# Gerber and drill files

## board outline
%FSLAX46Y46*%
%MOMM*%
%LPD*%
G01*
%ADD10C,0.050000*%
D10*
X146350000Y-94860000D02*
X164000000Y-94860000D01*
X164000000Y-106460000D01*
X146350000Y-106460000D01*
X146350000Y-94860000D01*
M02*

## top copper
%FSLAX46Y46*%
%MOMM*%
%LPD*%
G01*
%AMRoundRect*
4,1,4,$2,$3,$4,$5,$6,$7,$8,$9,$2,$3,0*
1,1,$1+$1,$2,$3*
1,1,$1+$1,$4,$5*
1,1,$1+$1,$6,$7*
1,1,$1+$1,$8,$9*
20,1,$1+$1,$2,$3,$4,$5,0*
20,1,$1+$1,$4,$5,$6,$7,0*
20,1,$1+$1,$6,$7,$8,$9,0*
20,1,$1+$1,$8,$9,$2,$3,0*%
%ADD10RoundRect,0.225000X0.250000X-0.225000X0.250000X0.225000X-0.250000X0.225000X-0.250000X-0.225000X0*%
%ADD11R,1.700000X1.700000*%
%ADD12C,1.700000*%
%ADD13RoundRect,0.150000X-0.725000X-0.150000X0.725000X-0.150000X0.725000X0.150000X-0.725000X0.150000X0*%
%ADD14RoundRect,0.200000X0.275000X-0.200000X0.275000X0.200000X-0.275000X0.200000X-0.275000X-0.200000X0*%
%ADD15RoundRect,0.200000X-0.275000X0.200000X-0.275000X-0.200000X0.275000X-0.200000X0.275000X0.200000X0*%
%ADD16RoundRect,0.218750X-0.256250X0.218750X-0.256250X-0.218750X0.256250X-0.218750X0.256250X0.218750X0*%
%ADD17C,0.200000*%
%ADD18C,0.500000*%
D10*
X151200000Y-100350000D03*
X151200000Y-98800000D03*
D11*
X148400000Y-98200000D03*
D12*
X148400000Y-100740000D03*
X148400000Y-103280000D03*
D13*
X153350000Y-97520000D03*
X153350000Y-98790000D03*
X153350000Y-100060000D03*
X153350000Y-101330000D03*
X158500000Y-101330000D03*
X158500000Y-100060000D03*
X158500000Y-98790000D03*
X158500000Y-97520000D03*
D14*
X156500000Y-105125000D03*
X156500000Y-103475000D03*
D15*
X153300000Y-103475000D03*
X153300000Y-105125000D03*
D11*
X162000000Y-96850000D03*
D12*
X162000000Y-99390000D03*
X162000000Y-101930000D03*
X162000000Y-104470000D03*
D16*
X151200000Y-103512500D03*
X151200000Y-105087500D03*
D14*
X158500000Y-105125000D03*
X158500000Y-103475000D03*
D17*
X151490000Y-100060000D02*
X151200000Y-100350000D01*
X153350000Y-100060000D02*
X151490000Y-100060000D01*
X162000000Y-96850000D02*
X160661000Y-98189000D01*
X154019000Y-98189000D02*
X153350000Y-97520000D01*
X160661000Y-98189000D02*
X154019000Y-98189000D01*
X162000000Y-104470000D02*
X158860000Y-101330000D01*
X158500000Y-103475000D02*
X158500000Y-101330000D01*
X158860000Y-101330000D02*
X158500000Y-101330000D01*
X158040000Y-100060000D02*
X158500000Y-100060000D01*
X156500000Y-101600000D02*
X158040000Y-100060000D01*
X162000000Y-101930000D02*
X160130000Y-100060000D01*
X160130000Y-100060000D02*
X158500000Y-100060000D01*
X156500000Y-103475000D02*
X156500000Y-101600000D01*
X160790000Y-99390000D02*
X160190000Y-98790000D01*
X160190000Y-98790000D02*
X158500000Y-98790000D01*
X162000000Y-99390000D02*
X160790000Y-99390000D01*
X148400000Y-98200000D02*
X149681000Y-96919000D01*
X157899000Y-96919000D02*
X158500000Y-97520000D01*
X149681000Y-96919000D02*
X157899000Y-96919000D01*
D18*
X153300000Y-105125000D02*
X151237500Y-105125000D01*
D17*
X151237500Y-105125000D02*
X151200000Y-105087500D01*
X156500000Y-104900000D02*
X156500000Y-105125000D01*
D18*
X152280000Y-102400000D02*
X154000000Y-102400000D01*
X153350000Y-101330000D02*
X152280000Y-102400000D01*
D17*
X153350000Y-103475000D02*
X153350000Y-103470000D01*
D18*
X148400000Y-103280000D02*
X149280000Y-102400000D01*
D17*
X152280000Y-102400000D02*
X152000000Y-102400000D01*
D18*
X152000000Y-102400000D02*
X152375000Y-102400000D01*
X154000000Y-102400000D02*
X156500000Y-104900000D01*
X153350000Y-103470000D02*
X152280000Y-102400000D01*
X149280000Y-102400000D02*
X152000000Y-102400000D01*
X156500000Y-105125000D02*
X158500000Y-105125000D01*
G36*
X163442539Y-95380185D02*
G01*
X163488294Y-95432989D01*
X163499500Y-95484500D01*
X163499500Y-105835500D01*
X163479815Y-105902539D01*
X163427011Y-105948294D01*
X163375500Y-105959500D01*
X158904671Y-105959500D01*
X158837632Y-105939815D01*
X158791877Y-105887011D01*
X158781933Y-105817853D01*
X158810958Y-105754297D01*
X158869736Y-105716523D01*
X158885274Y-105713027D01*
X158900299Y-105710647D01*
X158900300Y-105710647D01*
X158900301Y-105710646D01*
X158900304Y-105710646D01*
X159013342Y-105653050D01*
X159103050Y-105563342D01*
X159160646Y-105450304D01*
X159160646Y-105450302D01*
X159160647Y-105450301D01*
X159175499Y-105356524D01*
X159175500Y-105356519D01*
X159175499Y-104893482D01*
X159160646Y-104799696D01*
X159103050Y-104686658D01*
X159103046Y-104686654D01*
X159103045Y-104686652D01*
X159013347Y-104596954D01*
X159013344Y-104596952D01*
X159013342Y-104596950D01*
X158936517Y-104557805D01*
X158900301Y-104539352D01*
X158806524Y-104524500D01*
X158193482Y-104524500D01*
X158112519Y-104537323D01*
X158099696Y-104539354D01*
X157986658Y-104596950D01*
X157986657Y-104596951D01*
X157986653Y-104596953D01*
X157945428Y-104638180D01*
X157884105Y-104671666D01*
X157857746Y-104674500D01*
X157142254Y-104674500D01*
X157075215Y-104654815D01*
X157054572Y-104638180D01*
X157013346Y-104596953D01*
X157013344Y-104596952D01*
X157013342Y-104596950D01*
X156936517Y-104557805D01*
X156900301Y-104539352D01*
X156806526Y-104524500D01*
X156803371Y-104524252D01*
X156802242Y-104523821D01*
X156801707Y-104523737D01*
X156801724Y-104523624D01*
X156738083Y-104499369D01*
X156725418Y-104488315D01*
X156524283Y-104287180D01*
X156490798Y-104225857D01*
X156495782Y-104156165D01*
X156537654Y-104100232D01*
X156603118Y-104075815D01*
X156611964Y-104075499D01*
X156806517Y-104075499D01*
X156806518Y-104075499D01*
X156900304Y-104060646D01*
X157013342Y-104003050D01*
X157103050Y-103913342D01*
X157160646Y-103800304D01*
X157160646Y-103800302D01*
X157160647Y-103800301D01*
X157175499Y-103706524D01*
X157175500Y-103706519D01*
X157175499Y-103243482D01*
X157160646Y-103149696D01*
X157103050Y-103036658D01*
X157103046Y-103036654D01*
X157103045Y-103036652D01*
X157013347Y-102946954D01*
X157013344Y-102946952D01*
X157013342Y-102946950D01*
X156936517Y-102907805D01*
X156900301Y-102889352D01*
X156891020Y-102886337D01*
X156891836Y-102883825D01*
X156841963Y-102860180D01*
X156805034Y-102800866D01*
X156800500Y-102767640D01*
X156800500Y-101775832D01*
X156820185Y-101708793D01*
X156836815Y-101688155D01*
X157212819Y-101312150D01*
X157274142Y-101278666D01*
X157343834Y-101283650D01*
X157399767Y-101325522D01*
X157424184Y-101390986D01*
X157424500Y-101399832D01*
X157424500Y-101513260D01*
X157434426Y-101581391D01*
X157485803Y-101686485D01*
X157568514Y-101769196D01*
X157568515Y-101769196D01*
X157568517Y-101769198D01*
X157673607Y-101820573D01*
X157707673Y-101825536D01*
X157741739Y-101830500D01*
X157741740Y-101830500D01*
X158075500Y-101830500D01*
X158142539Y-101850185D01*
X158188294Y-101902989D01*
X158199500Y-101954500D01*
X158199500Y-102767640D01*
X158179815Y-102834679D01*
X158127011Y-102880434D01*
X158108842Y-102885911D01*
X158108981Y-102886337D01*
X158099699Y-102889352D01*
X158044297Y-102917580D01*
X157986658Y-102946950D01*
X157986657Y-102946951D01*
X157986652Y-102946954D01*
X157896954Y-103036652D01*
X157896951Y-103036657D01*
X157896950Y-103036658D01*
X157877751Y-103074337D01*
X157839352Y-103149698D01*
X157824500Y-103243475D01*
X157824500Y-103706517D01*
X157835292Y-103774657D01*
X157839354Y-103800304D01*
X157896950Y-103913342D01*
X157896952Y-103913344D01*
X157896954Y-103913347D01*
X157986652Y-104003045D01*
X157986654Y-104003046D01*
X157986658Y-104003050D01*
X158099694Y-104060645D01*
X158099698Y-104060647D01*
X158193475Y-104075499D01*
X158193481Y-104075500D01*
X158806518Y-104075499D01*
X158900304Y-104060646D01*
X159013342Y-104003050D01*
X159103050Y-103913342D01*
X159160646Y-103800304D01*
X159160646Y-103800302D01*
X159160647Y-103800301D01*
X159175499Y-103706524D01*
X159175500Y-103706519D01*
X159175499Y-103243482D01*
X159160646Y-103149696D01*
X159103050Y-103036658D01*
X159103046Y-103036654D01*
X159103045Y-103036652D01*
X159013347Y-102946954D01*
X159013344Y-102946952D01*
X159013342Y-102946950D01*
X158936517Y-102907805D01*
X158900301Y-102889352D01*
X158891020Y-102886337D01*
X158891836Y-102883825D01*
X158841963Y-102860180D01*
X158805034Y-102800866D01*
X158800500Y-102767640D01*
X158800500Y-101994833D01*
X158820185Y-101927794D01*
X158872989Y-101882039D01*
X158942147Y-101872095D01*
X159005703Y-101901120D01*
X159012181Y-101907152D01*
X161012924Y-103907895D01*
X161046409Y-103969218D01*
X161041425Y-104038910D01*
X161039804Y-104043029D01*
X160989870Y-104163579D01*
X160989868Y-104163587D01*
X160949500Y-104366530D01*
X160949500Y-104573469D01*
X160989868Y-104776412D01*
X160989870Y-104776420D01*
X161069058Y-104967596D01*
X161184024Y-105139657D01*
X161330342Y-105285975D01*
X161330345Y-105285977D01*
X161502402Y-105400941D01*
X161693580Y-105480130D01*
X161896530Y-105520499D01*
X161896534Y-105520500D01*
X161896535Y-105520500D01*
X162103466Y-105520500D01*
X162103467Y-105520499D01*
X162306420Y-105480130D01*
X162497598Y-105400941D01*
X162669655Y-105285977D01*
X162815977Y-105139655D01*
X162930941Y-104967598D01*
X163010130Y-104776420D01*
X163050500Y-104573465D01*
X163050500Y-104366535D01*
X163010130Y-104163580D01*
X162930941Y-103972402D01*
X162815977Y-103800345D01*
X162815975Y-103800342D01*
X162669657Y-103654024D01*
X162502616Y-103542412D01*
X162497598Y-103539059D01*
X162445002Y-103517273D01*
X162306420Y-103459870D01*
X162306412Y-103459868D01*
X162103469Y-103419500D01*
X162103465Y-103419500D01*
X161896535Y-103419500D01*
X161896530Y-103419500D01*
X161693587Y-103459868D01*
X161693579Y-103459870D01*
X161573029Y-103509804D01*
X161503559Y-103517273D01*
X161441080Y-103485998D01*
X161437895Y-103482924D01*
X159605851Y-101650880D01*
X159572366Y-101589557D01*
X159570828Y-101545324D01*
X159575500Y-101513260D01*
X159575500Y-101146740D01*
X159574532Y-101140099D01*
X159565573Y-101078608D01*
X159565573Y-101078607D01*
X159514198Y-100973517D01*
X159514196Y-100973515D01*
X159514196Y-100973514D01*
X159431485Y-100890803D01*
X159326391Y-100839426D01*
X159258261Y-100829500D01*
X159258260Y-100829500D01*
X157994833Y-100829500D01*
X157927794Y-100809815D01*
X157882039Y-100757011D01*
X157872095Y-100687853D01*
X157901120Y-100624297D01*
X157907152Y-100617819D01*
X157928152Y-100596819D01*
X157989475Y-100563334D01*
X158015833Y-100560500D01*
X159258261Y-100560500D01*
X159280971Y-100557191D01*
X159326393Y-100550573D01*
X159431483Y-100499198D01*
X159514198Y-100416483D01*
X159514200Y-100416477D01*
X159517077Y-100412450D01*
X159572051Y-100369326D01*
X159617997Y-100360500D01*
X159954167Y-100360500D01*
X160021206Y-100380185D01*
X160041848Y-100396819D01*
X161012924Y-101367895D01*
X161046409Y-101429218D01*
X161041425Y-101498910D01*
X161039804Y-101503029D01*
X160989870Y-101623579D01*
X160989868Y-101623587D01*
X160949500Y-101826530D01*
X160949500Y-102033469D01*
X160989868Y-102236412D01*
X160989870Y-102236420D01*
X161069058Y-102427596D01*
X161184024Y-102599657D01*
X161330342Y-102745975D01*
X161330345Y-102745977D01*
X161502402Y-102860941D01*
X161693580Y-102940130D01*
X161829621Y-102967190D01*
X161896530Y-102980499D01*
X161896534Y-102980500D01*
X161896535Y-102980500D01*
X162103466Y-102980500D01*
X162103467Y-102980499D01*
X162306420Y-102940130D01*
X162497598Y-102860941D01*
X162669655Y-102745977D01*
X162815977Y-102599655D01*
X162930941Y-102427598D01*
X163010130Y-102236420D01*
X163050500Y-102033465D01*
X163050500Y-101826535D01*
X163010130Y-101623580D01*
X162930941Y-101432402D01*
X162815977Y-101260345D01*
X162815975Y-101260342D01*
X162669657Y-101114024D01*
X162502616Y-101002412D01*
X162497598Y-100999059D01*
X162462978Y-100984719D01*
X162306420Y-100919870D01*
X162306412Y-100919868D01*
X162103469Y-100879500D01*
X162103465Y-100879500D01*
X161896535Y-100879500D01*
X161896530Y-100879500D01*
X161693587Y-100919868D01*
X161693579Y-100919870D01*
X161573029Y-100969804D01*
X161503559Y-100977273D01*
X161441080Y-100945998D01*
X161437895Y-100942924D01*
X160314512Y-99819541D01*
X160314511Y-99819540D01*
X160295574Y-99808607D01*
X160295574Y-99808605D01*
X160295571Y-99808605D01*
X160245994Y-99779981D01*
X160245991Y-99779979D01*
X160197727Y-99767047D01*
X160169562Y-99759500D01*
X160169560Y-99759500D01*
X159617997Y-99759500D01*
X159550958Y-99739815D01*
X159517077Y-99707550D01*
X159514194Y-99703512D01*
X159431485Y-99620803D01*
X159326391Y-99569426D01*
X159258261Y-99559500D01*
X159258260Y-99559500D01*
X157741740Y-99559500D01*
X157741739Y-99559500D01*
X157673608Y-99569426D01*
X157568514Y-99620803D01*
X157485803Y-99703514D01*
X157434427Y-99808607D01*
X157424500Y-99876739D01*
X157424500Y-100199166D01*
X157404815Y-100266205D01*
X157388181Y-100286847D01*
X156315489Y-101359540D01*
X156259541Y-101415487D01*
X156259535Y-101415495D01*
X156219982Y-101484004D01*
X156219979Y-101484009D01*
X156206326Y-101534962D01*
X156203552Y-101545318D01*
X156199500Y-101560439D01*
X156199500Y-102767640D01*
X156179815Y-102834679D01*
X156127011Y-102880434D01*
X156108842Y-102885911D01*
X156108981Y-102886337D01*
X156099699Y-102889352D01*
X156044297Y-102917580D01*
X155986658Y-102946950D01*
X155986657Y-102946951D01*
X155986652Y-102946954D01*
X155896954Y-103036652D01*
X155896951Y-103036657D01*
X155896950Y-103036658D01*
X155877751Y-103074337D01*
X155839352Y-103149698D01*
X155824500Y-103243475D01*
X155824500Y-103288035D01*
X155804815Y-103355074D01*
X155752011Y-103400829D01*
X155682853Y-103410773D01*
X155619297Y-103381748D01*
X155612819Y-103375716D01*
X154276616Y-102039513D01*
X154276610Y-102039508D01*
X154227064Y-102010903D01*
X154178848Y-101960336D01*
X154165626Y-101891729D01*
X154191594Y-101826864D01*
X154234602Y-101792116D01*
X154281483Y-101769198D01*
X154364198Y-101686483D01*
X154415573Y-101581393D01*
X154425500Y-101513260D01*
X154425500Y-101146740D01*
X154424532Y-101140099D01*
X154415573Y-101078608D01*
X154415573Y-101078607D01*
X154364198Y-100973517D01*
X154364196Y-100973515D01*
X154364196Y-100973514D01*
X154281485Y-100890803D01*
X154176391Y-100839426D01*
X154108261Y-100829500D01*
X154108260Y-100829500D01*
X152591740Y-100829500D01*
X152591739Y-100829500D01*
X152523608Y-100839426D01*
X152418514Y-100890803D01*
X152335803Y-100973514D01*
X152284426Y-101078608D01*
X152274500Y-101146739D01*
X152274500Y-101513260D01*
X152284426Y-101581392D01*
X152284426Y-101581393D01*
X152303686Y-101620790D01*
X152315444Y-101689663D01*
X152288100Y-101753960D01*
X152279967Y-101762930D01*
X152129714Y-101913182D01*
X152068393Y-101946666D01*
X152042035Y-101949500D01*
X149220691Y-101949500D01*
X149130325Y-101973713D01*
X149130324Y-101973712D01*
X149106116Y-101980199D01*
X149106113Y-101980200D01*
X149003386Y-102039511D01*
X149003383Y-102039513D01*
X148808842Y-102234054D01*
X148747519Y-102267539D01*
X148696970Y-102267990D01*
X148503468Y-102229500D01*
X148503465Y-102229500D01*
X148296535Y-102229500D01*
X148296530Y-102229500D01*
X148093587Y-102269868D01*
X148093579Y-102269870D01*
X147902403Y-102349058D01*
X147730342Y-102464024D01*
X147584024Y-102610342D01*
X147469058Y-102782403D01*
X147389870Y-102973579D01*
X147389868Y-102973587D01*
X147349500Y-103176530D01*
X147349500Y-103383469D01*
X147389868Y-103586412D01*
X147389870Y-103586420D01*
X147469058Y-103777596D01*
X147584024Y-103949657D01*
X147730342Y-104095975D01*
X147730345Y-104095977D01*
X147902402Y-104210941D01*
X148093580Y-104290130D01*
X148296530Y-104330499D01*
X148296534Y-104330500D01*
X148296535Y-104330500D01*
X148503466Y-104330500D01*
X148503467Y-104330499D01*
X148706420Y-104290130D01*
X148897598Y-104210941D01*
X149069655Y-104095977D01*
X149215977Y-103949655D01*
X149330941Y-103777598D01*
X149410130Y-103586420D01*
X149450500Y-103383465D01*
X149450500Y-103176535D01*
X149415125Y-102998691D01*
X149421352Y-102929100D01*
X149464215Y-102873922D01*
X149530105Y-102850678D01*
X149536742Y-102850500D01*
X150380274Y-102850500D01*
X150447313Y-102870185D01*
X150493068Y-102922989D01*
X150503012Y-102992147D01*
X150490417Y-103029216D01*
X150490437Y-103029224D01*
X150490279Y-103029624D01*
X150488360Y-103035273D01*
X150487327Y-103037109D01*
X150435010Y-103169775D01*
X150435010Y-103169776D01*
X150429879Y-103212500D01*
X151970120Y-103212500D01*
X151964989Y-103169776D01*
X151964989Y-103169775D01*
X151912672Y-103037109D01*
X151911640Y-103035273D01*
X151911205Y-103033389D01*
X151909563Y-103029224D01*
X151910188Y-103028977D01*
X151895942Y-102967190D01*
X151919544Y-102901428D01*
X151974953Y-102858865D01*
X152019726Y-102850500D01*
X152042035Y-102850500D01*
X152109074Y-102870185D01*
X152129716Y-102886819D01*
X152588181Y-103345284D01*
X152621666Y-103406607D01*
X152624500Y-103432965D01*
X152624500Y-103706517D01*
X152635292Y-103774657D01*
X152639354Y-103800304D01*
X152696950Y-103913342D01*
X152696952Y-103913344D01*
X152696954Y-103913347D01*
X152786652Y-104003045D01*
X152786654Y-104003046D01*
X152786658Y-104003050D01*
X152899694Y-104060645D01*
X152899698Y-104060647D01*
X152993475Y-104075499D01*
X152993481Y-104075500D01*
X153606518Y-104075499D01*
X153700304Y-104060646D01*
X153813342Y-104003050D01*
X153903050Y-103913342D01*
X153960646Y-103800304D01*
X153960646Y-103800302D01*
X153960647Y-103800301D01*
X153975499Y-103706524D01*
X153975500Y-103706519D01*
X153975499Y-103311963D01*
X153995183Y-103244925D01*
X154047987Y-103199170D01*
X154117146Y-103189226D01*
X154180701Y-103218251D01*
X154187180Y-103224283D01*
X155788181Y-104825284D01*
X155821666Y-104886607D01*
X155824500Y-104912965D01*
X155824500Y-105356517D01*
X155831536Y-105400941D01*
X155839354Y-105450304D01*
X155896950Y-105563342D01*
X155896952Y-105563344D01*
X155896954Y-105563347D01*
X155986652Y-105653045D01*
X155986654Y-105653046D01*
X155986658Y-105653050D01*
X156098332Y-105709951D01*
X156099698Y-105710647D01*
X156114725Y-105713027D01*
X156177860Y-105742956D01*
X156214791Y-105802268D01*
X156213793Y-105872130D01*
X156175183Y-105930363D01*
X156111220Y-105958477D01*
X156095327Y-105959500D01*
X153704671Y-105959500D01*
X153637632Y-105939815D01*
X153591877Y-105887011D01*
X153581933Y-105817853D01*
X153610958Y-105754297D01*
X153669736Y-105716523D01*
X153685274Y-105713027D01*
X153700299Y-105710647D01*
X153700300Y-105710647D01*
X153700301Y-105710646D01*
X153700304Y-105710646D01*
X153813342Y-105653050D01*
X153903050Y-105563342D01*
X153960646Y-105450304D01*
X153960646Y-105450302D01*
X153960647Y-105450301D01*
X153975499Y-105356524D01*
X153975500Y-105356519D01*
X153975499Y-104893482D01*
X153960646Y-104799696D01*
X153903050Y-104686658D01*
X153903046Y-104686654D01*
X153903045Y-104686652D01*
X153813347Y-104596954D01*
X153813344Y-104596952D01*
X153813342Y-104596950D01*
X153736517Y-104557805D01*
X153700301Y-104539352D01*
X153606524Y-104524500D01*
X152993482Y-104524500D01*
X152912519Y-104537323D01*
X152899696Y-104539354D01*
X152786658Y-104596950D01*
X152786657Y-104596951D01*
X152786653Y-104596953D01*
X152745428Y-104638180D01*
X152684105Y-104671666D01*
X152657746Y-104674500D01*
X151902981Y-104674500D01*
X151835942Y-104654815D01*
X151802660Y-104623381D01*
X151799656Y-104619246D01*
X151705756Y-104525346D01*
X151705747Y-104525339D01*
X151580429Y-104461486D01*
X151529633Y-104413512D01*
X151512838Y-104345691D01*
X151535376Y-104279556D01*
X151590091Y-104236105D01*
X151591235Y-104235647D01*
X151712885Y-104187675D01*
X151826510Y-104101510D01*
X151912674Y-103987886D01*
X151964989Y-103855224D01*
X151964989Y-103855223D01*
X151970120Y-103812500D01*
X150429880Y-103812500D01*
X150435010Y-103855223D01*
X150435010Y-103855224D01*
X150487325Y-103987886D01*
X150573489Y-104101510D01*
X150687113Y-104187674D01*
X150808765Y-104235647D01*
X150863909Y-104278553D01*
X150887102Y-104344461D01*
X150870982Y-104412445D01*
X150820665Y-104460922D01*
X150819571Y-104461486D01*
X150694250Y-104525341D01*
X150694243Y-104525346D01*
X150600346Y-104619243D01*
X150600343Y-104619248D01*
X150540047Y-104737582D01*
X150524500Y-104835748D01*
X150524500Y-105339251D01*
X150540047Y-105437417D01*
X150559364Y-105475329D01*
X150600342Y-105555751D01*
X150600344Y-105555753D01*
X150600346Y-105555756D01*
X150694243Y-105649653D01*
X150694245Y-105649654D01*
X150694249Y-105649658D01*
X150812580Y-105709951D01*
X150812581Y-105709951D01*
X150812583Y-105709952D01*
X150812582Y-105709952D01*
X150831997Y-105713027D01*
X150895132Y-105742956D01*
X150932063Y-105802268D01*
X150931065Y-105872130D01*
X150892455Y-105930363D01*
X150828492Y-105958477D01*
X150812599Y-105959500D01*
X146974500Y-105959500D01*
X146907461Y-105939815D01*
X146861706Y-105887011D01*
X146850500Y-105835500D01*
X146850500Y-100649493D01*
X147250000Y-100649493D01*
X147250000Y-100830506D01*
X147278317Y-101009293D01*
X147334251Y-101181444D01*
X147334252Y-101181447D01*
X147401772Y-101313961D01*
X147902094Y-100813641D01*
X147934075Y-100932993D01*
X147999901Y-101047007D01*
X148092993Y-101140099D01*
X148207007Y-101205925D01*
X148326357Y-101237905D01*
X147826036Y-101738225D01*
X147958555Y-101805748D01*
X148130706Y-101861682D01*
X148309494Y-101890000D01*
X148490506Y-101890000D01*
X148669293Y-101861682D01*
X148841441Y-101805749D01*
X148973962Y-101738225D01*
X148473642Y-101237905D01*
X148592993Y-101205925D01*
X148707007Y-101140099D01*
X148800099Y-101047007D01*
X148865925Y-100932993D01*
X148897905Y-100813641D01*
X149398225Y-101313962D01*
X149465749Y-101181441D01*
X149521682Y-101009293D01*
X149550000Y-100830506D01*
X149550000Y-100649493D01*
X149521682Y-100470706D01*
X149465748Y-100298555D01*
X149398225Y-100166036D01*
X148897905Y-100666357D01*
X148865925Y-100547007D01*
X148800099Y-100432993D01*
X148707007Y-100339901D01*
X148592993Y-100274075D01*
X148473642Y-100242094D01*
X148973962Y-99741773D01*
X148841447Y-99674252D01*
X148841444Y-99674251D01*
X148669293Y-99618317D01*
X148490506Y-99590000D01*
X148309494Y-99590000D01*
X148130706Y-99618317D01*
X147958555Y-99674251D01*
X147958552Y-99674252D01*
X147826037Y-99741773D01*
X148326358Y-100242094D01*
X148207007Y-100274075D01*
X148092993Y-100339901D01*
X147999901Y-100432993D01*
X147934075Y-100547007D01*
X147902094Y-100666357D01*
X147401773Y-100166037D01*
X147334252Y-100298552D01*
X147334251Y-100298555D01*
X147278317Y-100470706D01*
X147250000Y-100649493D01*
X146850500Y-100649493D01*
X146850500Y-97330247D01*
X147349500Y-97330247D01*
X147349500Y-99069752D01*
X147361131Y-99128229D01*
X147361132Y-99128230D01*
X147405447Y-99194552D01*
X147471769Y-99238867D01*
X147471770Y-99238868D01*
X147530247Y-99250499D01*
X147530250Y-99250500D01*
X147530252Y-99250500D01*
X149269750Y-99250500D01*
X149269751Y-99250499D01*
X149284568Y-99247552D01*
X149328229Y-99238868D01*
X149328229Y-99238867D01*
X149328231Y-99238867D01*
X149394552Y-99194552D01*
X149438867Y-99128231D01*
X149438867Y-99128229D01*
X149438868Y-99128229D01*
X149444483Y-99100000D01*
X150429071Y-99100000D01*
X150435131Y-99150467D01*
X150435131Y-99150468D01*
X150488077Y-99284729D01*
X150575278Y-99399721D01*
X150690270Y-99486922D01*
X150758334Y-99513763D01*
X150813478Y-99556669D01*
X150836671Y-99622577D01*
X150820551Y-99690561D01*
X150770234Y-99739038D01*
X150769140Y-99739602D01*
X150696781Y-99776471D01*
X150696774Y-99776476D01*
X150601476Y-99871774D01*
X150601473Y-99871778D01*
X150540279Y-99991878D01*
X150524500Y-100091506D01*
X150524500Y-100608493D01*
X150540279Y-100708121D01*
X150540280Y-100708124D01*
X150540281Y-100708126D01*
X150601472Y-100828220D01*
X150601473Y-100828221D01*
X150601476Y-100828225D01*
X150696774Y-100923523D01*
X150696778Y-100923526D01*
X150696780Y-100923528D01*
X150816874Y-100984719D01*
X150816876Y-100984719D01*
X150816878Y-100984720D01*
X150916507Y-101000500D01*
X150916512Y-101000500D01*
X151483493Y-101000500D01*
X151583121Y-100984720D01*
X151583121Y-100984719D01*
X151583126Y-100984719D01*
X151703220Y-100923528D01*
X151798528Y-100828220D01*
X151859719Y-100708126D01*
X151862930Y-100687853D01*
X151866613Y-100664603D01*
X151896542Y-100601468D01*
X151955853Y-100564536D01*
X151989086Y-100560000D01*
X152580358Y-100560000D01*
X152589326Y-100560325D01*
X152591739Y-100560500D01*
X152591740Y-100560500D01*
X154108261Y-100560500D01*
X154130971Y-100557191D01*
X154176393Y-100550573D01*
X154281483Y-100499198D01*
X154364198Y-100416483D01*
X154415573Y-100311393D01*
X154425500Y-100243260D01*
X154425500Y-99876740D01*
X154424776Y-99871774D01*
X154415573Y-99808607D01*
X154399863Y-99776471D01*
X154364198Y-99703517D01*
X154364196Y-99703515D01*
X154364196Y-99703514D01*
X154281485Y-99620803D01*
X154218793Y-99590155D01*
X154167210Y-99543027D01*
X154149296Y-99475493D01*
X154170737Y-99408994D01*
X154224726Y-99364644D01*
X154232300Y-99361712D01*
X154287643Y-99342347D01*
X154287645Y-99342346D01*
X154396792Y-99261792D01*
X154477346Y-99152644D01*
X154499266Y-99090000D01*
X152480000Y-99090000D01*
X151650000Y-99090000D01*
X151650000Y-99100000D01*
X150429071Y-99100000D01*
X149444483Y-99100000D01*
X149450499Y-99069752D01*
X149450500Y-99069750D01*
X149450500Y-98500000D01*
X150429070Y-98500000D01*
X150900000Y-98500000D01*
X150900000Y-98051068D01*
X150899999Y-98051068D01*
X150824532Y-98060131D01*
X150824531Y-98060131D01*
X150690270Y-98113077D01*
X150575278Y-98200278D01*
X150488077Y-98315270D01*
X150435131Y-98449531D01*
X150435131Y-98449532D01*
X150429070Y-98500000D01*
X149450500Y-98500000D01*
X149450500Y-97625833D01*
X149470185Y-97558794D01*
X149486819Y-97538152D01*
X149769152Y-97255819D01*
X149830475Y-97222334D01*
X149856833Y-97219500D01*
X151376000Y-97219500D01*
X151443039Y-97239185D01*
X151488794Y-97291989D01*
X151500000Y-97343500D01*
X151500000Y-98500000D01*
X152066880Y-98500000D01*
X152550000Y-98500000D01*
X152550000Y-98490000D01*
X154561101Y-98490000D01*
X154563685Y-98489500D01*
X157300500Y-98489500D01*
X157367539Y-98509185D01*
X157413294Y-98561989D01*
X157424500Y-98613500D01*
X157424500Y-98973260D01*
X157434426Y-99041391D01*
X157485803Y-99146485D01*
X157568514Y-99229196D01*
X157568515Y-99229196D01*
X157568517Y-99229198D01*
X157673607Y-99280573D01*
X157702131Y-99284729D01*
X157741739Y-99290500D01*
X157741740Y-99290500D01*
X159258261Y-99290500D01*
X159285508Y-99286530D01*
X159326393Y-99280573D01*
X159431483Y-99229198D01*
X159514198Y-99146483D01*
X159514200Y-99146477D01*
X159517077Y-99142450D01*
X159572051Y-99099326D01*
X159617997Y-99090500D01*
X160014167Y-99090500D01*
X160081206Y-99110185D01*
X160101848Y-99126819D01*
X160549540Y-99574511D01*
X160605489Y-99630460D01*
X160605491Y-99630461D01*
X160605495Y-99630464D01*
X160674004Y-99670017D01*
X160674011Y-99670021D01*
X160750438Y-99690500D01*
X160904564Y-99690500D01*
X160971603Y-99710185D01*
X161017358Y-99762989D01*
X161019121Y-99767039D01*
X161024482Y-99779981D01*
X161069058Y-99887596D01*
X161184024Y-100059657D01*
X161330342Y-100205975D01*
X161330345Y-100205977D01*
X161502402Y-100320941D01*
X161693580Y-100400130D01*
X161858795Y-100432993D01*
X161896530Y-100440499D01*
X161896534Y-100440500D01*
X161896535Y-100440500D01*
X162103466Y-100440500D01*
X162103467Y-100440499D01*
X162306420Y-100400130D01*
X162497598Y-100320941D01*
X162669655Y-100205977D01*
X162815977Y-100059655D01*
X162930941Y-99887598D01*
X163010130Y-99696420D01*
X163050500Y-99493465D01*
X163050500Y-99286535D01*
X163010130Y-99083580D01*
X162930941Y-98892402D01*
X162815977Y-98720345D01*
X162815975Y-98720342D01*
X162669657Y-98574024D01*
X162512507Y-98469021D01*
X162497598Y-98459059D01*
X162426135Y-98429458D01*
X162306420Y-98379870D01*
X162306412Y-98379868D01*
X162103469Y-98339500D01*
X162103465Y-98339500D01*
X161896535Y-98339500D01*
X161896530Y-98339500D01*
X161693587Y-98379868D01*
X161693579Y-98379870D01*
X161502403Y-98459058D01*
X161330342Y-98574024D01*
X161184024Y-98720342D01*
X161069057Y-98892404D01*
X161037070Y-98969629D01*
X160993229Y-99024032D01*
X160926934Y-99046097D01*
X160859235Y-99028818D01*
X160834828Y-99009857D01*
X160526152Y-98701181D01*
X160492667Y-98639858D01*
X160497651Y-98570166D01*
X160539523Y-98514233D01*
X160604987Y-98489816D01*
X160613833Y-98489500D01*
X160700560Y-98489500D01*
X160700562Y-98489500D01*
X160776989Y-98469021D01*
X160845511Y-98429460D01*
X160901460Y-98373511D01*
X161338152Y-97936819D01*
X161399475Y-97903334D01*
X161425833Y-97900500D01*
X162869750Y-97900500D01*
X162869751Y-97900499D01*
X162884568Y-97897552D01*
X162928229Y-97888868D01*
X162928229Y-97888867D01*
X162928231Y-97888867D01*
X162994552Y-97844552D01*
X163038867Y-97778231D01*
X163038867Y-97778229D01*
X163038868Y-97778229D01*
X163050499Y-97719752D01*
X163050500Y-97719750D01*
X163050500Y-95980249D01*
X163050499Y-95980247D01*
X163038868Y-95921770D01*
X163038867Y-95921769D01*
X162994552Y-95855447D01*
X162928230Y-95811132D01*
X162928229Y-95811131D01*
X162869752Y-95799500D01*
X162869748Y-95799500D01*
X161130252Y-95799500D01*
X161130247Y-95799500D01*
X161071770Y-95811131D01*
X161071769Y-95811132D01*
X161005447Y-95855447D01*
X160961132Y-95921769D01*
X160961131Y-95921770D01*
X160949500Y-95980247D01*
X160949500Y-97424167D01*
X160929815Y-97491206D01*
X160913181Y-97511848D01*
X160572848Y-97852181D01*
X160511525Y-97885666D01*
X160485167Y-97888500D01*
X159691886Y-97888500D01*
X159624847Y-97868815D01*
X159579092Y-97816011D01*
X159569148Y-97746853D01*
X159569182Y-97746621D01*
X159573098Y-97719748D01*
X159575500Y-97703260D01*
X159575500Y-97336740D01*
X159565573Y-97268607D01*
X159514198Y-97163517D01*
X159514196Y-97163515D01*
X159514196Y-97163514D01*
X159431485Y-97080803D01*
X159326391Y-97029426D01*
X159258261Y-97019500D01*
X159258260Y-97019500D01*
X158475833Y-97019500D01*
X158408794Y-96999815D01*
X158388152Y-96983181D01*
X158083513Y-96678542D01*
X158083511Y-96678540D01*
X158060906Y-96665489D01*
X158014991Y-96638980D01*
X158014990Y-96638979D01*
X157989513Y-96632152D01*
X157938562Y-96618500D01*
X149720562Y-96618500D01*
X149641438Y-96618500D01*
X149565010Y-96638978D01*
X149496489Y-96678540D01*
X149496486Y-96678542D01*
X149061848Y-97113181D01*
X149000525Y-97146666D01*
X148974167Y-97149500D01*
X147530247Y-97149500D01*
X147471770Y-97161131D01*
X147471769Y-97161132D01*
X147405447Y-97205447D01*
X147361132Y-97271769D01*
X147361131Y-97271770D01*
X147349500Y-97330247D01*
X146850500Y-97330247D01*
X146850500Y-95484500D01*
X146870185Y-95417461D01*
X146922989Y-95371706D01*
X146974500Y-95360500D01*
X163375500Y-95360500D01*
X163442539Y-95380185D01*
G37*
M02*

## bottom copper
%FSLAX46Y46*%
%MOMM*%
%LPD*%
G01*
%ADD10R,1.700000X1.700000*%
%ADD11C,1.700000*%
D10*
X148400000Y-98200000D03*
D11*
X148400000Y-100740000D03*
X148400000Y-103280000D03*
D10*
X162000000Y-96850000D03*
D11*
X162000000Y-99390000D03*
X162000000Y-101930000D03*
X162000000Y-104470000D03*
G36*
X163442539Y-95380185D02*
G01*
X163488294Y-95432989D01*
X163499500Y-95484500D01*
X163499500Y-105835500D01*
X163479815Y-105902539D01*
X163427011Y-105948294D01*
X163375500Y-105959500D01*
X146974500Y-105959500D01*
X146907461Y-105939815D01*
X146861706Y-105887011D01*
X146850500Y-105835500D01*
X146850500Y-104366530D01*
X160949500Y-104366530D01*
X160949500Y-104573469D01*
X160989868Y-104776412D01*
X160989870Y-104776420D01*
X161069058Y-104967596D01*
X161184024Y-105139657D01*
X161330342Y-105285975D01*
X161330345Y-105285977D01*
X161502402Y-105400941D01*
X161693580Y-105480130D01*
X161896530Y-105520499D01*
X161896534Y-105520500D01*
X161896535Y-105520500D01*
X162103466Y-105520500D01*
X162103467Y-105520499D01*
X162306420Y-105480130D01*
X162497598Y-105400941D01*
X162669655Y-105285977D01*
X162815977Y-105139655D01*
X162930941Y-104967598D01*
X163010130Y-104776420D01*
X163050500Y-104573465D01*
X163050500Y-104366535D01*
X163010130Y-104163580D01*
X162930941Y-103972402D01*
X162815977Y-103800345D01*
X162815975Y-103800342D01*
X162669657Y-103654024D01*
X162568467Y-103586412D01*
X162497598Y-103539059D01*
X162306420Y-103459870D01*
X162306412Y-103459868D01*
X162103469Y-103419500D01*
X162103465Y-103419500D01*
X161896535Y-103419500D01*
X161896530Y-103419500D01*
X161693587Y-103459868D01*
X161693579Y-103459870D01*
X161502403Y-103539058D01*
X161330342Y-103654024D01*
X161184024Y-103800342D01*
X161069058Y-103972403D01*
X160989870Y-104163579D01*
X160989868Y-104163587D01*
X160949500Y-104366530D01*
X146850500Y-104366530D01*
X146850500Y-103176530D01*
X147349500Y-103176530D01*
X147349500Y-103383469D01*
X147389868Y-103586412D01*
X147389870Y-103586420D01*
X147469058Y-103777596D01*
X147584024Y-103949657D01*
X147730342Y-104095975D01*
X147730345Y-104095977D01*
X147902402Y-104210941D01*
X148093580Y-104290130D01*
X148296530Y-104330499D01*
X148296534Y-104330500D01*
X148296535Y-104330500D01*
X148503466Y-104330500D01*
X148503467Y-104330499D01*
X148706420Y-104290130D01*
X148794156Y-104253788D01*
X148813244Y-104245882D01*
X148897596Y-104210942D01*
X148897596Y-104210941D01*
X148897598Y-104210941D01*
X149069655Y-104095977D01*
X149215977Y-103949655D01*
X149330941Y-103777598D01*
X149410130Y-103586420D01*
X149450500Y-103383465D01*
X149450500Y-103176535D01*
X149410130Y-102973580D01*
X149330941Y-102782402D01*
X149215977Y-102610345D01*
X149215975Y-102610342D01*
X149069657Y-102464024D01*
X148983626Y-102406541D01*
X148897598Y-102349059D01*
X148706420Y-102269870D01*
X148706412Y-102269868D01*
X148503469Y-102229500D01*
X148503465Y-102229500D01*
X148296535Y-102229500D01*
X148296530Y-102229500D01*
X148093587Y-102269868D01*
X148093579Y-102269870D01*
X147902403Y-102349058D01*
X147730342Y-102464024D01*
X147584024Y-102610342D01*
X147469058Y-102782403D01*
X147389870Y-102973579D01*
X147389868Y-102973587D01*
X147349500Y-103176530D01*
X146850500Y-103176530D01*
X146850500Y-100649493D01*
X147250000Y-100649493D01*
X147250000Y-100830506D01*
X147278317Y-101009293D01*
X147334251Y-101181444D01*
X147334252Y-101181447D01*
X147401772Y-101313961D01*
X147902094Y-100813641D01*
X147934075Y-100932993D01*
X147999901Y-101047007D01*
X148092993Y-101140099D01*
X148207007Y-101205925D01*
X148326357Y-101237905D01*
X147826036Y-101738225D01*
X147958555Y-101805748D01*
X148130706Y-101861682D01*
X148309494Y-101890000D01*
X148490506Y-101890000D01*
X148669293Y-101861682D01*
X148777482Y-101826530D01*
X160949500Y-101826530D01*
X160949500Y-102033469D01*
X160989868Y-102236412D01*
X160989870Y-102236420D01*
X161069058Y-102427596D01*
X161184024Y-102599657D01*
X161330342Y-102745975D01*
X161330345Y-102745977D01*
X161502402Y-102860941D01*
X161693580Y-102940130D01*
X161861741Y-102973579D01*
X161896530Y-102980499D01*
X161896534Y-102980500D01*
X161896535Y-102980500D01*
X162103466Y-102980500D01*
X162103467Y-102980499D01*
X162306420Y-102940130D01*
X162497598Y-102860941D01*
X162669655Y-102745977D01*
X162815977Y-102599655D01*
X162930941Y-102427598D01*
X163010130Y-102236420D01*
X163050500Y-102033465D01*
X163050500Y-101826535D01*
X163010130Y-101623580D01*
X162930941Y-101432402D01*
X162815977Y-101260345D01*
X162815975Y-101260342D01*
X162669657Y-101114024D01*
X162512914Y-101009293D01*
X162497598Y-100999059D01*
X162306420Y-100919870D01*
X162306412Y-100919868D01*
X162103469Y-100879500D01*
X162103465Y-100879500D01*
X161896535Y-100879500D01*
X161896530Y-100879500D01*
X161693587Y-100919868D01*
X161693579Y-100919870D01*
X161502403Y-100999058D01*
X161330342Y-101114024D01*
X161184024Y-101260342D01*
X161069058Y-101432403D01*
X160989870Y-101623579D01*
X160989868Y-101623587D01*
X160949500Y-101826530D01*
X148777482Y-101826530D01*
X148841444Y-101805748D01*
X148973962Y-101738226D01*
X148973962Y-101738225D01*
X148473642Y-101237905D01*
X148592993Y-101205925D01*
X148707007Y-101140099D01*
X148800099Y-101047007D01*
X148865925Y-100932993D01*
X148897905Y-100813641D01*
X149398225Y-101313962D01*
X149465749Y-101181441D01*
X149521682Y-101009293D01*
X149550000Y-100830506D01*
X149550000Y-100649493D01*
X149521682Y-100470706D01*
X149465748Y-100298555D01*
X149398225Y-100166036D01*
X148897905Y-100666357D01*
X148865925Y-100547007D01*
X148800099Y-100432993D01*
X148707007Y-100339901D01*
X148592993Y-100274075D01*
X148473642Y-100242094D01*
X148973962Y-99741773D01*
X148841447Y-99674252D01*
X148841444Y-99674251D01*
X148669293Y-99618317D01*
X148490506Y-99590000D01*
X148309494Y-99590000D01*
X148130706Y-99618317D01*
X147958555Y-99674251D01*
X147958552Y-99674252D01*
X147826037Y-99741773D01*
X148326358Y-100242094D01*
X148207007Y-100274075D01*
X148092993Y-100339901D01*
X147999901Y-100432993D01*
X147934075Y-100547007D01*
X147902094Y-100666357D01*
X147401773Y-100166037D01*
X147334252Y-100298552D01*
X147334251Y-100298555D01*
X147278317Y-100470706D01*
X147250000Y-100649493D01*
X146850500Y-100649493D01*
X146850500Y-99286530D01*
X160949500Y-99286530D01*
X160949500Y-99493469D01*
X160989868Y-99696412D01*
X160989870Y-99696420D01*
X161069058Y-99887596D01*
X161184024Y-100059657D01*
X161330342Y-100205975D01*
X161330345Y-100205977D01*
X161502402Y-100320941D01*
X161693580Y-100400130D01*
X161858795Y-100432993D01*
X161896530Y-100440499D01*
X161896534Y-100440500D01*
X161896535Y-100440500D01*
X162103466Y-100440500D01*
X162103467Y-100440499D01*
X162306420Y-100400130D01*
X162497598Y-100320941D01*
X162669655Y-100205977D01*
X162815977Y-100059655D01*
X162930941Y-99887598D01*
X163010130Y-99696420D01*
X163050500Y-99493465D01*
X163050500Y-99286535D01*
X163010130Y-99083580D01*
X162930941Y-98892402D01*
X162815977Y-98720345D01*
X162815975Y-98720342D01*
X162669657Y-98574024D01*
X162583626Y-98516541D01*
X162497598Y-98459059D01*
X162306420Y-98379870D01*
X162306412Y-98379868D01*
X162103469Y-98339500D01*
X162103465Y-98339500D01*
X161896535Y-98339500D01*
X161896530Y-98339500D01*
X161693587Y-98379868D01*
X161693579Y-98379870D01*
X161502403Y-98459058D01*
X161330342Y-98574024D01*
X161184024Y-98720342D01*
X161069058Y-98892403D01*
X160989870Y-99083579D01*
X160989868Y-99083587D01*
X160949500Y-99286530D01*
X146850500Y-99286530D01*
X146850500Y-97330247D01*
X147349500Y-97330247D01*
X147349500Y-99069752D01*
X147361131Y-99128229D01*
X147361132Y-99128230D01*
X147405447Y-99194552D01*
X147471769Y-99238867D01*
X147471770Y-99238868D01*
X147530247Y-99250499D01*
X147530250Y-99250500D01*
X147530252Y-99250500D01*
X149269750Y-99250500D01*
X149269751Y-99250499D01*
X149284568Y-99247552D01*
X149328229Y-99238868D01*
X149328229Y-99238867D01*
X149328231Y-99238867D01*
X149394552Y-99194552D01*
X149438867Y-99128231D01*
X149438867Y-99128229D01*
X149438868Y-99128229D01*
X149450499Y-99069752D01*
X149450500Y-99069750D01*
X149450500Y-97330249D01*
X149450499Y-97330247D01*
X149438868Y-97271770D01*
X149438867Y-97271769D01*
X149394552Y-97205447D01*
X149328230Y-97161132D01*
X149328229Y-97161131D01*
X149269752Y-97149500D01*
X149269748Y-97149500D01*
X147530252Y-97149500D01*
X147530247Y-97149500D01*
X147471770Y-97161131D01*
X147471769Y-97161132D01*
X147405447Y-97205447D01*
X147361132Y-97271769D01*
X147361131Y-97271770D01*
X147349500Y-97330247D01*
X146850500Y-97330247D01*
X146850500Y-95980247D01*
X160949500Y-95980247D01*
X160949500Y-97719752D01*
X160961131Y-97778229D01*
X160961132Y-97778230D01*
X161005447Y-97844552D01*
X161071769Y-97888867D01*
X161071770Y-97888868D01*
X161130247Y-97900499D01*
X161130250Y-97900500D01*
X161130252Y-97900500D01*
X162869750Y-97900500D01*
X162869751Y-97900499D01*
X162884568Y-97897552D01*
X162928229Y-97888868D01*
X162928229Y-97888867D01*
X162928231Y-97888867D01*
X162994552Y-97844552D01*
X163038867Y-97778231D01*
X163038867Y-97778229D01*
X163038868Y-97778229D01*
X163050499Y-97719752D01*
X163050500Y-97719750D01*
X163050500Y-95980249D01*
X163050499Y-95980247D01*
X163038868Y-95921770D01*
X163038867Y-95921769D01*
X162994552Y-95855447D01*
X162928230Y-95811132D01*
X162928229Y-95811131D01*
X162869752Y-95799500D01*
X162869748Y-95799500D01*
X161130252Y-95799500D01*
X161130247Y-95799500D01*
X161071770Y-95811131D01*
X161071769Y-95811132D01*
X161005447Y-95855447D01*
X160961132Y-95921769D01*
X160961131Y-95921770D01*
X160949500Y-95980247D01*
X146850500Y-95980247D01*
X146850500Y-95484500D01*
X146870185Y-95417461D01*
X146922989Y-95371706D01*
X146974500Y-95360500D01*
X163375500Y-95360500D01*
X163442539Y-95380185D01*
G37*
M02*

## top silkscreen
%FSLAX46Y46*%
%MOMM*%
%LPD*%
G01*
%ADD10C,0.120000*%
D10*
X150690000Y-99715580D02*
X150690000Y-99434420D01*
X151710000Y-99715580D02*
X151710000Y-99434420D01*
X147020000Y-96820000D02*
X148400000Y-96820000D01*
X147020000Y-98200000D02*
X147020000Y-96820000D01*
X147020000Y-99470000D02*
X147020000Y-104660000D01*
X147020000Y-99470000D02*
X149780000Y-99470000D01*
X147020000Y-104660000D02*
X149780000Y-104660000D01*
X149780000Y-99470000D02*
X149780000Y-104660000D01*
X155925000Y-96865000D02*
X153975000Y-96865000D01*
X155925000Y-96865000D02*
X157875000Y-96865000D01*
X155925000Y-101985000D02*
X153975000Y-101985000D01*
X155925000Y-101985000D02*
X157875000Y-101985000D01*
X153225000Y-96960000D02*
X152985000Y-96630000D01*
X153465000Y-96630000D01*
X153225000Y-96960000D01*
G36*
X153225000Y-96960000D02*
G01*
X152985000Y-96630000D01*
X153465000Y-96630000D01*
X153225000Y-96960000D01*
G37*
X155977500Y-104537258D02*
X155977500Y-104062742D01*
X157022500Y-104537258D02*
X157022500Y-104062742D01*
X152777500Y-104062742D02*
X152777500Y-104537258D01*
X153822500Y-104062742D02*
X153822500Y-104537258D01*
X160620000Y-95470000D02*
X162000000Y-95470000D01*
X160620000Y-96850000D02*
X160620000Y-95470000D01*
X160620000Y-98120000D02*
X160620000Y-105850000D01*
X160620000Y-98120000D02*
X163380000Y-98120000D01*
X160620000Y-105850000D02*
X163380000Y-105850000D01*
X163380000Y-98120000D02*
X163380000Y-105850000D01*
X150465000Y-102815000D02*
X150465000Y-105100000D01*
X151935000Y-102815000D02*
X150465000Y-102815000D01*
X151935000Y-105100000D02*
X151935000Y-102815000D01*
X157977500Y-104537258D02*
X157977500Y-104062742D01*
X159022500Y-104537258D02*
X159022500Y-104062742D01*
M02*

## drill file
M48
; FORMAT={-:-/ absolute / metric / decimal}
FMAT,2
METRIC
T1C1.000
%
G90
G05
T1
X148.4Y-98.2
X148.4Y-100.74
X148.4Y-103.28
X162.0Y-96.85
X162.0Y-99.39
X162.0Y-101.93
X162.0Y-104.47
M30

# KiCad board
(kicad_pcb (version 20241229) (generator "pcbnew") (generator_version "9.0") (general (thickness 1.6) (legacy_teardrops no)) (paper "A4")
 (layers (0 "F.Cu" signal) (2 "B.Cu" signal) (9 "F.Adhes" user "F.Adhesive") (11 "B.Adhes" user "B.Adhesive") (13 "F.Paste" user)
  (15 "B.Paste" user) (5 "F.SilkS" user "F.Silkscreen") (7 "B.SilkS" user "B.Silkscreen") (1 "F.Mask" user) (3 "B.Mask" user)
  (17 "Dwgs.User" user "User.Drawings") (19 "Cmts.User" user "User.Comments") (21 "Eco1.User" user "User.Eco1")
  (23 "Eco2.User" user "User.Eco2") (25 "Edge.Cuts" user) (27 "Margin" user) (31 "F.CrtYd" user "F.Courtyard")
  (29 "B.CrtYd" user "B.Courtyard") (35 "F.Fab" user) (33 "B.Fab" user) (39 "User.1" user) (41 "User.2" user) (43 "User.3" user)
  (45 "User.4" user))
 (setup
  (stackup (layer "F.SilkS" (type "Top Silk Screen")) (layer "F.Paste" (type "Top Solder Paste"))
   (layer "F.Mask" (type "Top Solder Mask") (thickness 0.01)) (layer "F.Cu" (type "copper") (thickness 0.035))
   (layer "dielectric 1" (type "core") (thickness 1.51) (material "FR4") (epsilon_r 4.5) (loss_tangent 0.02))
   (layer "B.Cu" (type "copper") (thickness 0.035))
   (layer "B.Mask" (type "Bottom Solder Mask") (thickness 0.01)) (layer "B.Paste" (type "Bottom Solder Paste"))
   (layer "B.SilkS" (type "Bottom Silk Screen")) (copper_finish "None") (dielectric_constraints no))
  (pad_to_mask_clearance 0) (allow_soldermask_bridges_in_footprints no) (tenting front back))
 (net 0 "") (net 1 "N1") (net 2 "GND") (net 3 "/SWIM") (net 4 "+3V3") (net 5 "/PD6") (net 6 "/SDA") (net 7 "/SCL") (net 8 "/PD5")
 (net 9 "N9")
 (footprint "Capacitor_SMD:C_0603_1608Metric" (layer "F.Cu") (at 151.2 99.575 90)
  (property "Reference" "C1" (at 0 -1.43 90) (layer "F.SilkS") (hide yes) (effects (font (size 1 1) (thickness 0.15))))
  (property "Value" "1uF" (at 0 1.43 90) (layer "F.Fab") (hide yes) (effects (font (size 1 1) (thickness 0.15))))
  (fp_line (start -0.14058 -0.51) (end 0.14058 -0.51) (stroke (width 0.12) (type solid)) (layer "F.SilkS"))
  (fp_line (start -0.14058 0.51) (end 0.14058 0.51) (stroke (width 0.12) (type solid)) (layer "F.SilkS"))
  (pad "1" smd roundrect (at -0.775 0 90) (size 0.9 0.95) (layers "F.Cu" "F.Mask" "F.Paste") (roundrect_rratio 0.25) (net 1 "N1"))
  (pad "2" smd roundrect (at 0.775 0 90) (size 0.9 0.95) (layers "F.Cu" "F.Mask" "F.Paste") (roundrect_rratio 0.25) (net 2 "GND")))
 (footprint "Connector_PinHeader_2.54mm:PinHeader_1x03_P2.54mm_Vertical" (layer "F.Cu") (at 148.4 98.2)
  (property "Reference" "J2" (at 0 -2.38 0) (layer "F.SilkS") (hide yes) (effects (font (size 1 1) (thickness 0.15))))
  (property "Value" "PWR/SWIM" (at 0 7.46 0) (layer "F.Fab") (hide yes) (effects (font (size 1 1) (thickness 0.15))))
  (fp_line (start -1.38 -1.38) (end 0 -1.38) (stroke (width 0.12) (type solid)) (layer "F.SilkS"))
  (fp_line (start -1.38 0) (end -1.38 -1.38) (stroke (width 0.12) (type solid)) (layer "F.SilkS"))
  (fp_line (start -1.38 1.27) (end -1.38 6.46) (stroke (width 0.12) (type solid)) (layer "F.SilkS"))
  (fp_line (start -1.38 1.27) (end 1.38 1.27) (stroke (width 0.12) (type solid)) (layer "F.SilkS"))
  (fp_line (start -1.38 6.46) (end 1.38 6.46) (stroke (width 0.12) (type solid)) (layer "F.SilkS"))
  (fp_line (start 1.38 1.27) (end 1.38 6.46) (stroke (width 0.12) (type solid)) (layer "F.SilkS"))
  (pad "1" thru_hole rect (at 0 0) (size 1.7 1.7) (drill 1) (layers "*.Cu" "*.Mask") (remove_unused_layers no) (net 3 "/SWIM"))
  (pad "2" thru_hole circle (at 0 2.54) (size 1.7 1.7) (drill 1) (layers "*.Cu" "*.Mask") (remove_unused_layers no) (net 2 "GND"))
  (pad "3" thru_hole circle (at 0 5.08) (size 1.7 1.7) (drill 1) (layers "*.Cu" "*.Mask") (remove_unused_layers no) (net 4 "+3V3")))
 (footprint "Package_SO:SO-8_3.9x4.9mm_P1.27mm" (layer "F.Cu") (at 155.925 99.425)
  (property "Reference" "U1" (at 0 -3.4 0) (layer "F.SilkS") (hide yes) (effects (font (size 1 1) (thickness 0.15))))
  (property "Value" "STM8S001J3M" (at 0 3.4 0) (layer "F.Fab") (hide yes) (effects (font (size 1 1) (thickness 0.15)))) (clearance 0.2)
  (fp_line (start 0 -2.56) (end -1.95 -2.56) (stroke (width 0.12) (type solid)) (layer "F.SilkS"))
  (fp_line (start 0 -2.56) (end 1.95 -2.56) (stroke (width 0.12) (type solid)) (layer "F.SilkS"))
  (fp_line (start 0 2.56) (end -1.95 2.56) (stroke (width 0.12) (type solid)) (layer "F.SilkS"))
  (fp_line (start 0 2.56) (end 1.95 2.56) (stroke (width 0.12) (type solid)) (layer "F.SilkS"))
  (fp_poly (pts (xy -2.7 -2.465) (xy -2.94 -2.795) (xy -2.46 -2.795)) (stroke (width 0.12) (type solid)) (fill yes) (layer "F.SilkS"))
  (pad "1" smd roundrect (at -2.575 -1.905) (size 1.75 0.6) (layers "F.Cu" "F.Mask" "F.Paste") (roundrect_rratio 0.25) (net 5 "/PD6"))
  (pad "2" smd roundrect (at -2.575 -0.635) (size 1.75 0.6) (layers "F.Cu" "F.Mask" "F.Paste") (roundrect_rratio 0.25) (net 2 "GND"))
  (pad "3" smd roundrect (at -2.575 0.635) (size 1.75 0.6) (layers "F.Cu" "F.Mask" "F.Paste") (roundrect_rratio 0.25) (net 1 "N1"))
  (pad "4" smd roundrect (at -2.575 1.905) (size 1.75 0.6) (layers "F.Cu" "F.Mask" "F.Paste") (roundrect_rratio 0.25) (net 4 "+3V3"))
  (pad "5" smd roundrect (at 2.575 1.905) (size 1.75 0.6) (layers "F.Cu" "F.Mask" "F.Paste") (roundrect_rratio 0.25) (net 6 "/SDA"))
  (pad "6" smd roundrect (at 2.575 0.635) (size 1.75 0.6) (layers "F.Cu" "F.Mask" "F.Paste") (roundrect_rratio 0.25) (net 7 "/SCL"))
  (pad "7" smd roundrect (at 2.575 -0.635) (size 1.75 0.6) (layers "F.Cu" "F.Mask" "F.Paste") (roundrect_rratio 0.25) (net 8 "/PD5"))
  (pad "8" smd roundrect (at 2.575 -1.905) (size 1.75 0.6) (layers "F.Cu" "F.Mask" "F.Paste") (roundrect_rratio 0.25) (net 3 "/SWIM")))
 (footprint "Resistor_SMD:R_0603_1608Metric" (layer "F.Cu") (at 156.5 104.3 90)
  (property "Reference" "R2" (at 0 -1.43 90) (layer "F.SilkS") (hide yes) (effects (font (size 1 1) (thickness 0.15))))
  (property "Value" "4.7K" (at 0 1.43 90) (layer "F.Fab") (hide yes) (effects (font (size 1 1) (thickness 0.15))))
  (fp_line (start -0.237258 -0.5225) (end 0.237258 -0.5225) (stroke (width 0.12) (type solid)) (layer "F.SilkS"))
  (fp_line (start -0.237258 0.5225) (end 0.237258 0.5225) (stroke (width 0.12) (type solid)) (layer "F.SilkS"))
  (pad "1" smd roundrect (at -0.825 0 90) (size 0.8 0.95) (layers "F.Cu" "F.Mask" "F.Paste") (roundrect_rratio 0.25) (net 4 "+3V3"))
  (pad "2" smd roundrect (at 0.825 0 90) (size 0.8 0.95) (layers "F.Cu" "F.Mask" "F.Paste") (roundrect_rratio 0.25) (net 7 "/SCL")))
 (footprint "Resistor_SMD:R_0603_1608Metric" (layer "F.Cu") (at 153.3 104.3 -90)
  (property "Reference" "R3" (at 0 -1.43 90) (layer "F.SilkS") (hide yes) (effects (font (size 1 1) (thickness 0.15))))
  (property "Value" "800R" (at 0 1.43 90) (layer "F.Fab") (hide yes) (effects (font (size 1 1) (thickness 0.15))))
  (fp_line (start -0.237258 0.5225) (end 0.237258 0.5225) (stroke (width 0.12) (type solid)) (layer "F.SilkS"))
  (fp_line (start -0.237258 -0.5225) (end 0.237258 -0.5225) (stroke (width 0.12) (type solid)) (layer "F.SilkS"))
  (pad "1" smd roundrect (at -0.825 0 270) (size 0.8 0.95) (layers "F.Cu" "F.Mask" "F.Paste") (roundrect_rratio 0.25) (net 4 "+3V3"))
  (pad "2" smd roundrect (at 0.825 0 270) (size 0.8 0.95) (layers "F.Cu" "F.Mask" "F.Paste") (roundrect_rratio 0.25) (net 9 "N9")))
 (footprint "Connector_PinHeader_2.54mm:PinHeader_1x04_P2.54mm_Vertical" (layer "F.Cu") (at 162 96.85)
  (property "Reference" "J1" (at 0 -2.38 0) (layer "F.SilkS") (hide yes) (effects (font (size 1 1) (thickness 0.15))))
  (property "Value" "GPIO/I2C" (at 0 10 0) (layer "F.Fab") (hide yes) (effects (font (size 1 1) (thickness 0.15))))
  (fp_line (start -1.38 -1.38) (end 0 -1.38) (stroke (width 0.12) (type solid)) (layer "F.SilkS"))
  (fp_line (start -1.38 0) (end -1.38 -1.38) (stroke (width 0.12) (type solid)) (layer "F.SilkS"))
  (fp_line (start -1.38 1.27) (end -1.38 9) (stroke (width 0.12) (type solid)) (layer "F.SilkS"))
  (fp_line (start -1.38 1.27) (end 1.38 1.27) (stroke (width 0.12) (type solid)) (layer "F.SilkS"))
  (fp_line (start -1.38 9) (end 1.38 9) (stroke (width 0.12) (type solid)) (layer "F.SilkS"))
  (fp_line (start 1.38 1.27) (end 1.38 9) (stroke (width 0.12) (type solid)) (layer "F.SilkS"))
  (pad "1" thru_hole rect (at 0 0) (size 1.7 1.7) (drill 1) (layers "*.Cu" "*.Mask") (remove_unused_layers no) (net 5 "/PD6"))
  (pad "2" thru_hole circle (at 0 2.54) (size 1.7 1.7) (drill 1) (layers "*.Cu" "*.Mask") (remove_unused_layers no) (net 8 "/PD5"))
  (pad "3" thru_hole circle (at 0 5.08) (size 1.7 1.7) (drill 1) (layers "*.Cu" "*.Mask") (remove_unused_layers no) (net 7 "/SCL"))
  (pad "4" thru_hole circle (at 0 7.62) (size 1.7 1.7) (drill 1) (layers "*.Cu" "*.Mask") (remove_unused_layers no) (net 6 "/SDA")))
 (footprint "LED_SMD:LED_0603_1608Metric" (layer "F.Cu") (at 151.2 104.3 -90)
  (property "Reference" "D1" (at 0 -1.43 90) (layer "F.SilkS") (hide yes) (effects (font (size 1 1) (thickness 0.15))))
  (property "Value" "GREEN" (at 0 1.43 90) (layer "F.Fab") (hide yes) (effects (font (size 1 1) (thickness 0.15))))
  (fp_line (start -1.485 0.735) (end 0.8 0.735) (stroke (width 0.12) (type solid)) (layer "F.SilkS"))
  (fp_line (start -1.485 -0.735) (end -1.485 0.735) (stroke (width 0.12) (type solid)) (layer "F.SilkS"))
  (fp_line (start 0.8 -0.735) (end -1.485 -0.735) (stroke (width 0.12) (type solid)) (layer "F.SilkS"))
  (pad "1" smd roundrect (at -0.7875 0 270) (size 0.875 0.95) (layers "F.Cu" "F.Mask" "F.Paste") (roundrect_rratio 0.25) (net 2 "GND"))
  (pad "2" smd roundrect (at 0.7875 0 270) (size 0.875 0.95) (layers "F.Cu" "F.Mask" "F.Paste") (roundrect_rratio 0.25) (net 9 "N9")))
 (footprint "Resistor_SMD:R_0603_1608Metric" (layer "F.Cu") (at 158.5 104.3 90)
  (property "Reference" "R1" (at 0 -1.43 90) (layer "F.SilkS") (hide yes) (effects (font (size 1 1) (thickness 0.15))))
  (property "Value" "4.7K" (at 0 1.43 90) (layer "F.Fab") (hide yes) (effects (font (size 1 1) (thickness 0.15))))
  (fp_line (start -0.237258 -0.5225) (end 0.237258 -0.5225) (stroke (width 0.12) (type solid)) (layer "F.SilkS"))
  (fp_line (start -0.237258 0.5225) (end 0.237258 0.5225) (stroke (width 0.12) (type solid)) (layer "F.SilkS"))
  (pad "1" smd roundrect (at -0.825 0 90) (size 0.8 0.95) (layers "F.Cu" "F.Mask" "F.Paste") (roundrect_rratio 0.25) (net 4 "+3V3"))
  (pad "2" smd roundrect (at 0.825 0 90) (size 0.8 0.95) (layers "F.Cu" "F.Mask" "F.Paste") (roundrect_rratio 0.25) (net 6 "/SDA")))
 (gr_rect (start 146.35 94.86) (end 164 106.46) (stroke (width 0.05) (type default)) (fill no) (layer "Edge.Cuts"))
 (segment (start 151.49 100.06) (end 151.2 100.35) (width 0.2) (layer "F.Cu") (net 1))
 (segment (start 153.35 100.06) (end 151.49 100.06) (width 0.2) (layer "F.Cu") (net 1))
 (segment (start 162 96.85) (end 160.661 98.189) (width 0.2) (layer "F.Cu") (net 5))
 (segment (start 154.019 98.189) (end 153.35 97.52) (width 0.2) (layer "F.Cu") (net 5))
 (segment (start 160.661 98.189) (end 154.019 98.189) (width 0.2) (layer "F.Cu") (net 5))
 (segment (start 162 104.47) (end 158.86 101.33) (width 0.2) (layer "F.Cu") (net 6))
 (segment (start 158.5 103.475) (end 158.5 101.33) (width 0.2) (layer "F.Cu") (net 6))
 (segment (start 158.86 101.33) (end 158.5 101.33) (width 0.2) (layer "F.Cu") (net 6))
 (segment (start 158.04 100.06) (end 158.5 100.06) (width 0.2) (layer "F.Cu") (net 7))
 (segment (start 156.5 101.6) (end 158.04 100.06) (width 0.2) (layer "F.Cu") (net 7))
 (segment (start 162 101.93) (end 160.13 100.06) (width 0.2) (layer "F.Cu") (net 7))
 (segment (start 160.13 100.06) (end 158.5 100.06) (width 0.2) (layer "F.Cu") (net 7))
 (segment (start 156.5 103.475) (end 156.5 101.6) (width 0.2) (layer "F.Cu") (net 7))
 (segment (start 160.79 99.39) (end 160.19 98.79) (width 0.2) (layer "F.Cu") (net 8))
 (segment (start 160.19 98.79) (end 158.5 98.79) (width 0.2) (layer "F.Cu") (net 8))
 (segment (start 162 99.39) (end 160.79 99.39) (width 0.2) (layer "F.Cu") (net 8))
 (segment (start 148.4 98.2) (end 149.681 96.919) (width 0.2) (layer "F.Cu") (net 3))
 (segment (start 157.899 96.919) (end 158.5 97.52) (width 0.2) (layer "F.Cu") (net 3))
 (segment (start 149.681 96.919) (end 157.899 96.919) (width 0.2) (layer "F.Cu") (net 3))
 (segment (start 153.3 105.125) (end 151.2375 105.125) (width 0.5) (layer "F.Cu") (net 9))
 (segment (start 151.2375 105.125) (end 151.2 105.0875) (width 0.2) (layer "F.Cu") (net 9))
 (segment (start 156.5 104.9) (end 156.5 105.125) (width 0.2) (layer "F.Cu") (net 4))
 (segment (start 152.28 102.4) (end 154 102.4) (width 0.5) (layer "F.Cu") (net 4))
 (segment (start 153.35 101.33) (end 152.28 102.4) (width 0.5) (layer "F.Cu") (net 4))
 (segment (start 153.35 103.475) (end 153.35 103.47) (width 0.2) (layer "F.Cu") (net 4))
 (segment (start 148.4 103.28) (end 149.28 102.4) (width 0.5) (layer "F.Cu") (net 4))
 (segment (start 152.28 102.4) (end 152 102.4) (width 0.2) (layer "F.Cu") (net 4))
 (segment (start 152 102.4) (end 152.375 102.4) (width 0.5) (layer "F.Cu") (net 4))
 (segment (start 154 102.4) (end 156.5 104.9) (width 0.5) (layer "F.Cu") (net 4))
 (segment (start 153.35 103.47) (end 152.28 102.4) (width 0.5) (layer "F.Cu") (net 4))
 (segment (start 149.28 102.4) (end 152 102.4) (width 0.5) (layer "F.Cu") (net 4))
 (segment (start 156.5 105.125) (end 158.5 105.125) (width 0.5) (layer "F.Cu") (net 4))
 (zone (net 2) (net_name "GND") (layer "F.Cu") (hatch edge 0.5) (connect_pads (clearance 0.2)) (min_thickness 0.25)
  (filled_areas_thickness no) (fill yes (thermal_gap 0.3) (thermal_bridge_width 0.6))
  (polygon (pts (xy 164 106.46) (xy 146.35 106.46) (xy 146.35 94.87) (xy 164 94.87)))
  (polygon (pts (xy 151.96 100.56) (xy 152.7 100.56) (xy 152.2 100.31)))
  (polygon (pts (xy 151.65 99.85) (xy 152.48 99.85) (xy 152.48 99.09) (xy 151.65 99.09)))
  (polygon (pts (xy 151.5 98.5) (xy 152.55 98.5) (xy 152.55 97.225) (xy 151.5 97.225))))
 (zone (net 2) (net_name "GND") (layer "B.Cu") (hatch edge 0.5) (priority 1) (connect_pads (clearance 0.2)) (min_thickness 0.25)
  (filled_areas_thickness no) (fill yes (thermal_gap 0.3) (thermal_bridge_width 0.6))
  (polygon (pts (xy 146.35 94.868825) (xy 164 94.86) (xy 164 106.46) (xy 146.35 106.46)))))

